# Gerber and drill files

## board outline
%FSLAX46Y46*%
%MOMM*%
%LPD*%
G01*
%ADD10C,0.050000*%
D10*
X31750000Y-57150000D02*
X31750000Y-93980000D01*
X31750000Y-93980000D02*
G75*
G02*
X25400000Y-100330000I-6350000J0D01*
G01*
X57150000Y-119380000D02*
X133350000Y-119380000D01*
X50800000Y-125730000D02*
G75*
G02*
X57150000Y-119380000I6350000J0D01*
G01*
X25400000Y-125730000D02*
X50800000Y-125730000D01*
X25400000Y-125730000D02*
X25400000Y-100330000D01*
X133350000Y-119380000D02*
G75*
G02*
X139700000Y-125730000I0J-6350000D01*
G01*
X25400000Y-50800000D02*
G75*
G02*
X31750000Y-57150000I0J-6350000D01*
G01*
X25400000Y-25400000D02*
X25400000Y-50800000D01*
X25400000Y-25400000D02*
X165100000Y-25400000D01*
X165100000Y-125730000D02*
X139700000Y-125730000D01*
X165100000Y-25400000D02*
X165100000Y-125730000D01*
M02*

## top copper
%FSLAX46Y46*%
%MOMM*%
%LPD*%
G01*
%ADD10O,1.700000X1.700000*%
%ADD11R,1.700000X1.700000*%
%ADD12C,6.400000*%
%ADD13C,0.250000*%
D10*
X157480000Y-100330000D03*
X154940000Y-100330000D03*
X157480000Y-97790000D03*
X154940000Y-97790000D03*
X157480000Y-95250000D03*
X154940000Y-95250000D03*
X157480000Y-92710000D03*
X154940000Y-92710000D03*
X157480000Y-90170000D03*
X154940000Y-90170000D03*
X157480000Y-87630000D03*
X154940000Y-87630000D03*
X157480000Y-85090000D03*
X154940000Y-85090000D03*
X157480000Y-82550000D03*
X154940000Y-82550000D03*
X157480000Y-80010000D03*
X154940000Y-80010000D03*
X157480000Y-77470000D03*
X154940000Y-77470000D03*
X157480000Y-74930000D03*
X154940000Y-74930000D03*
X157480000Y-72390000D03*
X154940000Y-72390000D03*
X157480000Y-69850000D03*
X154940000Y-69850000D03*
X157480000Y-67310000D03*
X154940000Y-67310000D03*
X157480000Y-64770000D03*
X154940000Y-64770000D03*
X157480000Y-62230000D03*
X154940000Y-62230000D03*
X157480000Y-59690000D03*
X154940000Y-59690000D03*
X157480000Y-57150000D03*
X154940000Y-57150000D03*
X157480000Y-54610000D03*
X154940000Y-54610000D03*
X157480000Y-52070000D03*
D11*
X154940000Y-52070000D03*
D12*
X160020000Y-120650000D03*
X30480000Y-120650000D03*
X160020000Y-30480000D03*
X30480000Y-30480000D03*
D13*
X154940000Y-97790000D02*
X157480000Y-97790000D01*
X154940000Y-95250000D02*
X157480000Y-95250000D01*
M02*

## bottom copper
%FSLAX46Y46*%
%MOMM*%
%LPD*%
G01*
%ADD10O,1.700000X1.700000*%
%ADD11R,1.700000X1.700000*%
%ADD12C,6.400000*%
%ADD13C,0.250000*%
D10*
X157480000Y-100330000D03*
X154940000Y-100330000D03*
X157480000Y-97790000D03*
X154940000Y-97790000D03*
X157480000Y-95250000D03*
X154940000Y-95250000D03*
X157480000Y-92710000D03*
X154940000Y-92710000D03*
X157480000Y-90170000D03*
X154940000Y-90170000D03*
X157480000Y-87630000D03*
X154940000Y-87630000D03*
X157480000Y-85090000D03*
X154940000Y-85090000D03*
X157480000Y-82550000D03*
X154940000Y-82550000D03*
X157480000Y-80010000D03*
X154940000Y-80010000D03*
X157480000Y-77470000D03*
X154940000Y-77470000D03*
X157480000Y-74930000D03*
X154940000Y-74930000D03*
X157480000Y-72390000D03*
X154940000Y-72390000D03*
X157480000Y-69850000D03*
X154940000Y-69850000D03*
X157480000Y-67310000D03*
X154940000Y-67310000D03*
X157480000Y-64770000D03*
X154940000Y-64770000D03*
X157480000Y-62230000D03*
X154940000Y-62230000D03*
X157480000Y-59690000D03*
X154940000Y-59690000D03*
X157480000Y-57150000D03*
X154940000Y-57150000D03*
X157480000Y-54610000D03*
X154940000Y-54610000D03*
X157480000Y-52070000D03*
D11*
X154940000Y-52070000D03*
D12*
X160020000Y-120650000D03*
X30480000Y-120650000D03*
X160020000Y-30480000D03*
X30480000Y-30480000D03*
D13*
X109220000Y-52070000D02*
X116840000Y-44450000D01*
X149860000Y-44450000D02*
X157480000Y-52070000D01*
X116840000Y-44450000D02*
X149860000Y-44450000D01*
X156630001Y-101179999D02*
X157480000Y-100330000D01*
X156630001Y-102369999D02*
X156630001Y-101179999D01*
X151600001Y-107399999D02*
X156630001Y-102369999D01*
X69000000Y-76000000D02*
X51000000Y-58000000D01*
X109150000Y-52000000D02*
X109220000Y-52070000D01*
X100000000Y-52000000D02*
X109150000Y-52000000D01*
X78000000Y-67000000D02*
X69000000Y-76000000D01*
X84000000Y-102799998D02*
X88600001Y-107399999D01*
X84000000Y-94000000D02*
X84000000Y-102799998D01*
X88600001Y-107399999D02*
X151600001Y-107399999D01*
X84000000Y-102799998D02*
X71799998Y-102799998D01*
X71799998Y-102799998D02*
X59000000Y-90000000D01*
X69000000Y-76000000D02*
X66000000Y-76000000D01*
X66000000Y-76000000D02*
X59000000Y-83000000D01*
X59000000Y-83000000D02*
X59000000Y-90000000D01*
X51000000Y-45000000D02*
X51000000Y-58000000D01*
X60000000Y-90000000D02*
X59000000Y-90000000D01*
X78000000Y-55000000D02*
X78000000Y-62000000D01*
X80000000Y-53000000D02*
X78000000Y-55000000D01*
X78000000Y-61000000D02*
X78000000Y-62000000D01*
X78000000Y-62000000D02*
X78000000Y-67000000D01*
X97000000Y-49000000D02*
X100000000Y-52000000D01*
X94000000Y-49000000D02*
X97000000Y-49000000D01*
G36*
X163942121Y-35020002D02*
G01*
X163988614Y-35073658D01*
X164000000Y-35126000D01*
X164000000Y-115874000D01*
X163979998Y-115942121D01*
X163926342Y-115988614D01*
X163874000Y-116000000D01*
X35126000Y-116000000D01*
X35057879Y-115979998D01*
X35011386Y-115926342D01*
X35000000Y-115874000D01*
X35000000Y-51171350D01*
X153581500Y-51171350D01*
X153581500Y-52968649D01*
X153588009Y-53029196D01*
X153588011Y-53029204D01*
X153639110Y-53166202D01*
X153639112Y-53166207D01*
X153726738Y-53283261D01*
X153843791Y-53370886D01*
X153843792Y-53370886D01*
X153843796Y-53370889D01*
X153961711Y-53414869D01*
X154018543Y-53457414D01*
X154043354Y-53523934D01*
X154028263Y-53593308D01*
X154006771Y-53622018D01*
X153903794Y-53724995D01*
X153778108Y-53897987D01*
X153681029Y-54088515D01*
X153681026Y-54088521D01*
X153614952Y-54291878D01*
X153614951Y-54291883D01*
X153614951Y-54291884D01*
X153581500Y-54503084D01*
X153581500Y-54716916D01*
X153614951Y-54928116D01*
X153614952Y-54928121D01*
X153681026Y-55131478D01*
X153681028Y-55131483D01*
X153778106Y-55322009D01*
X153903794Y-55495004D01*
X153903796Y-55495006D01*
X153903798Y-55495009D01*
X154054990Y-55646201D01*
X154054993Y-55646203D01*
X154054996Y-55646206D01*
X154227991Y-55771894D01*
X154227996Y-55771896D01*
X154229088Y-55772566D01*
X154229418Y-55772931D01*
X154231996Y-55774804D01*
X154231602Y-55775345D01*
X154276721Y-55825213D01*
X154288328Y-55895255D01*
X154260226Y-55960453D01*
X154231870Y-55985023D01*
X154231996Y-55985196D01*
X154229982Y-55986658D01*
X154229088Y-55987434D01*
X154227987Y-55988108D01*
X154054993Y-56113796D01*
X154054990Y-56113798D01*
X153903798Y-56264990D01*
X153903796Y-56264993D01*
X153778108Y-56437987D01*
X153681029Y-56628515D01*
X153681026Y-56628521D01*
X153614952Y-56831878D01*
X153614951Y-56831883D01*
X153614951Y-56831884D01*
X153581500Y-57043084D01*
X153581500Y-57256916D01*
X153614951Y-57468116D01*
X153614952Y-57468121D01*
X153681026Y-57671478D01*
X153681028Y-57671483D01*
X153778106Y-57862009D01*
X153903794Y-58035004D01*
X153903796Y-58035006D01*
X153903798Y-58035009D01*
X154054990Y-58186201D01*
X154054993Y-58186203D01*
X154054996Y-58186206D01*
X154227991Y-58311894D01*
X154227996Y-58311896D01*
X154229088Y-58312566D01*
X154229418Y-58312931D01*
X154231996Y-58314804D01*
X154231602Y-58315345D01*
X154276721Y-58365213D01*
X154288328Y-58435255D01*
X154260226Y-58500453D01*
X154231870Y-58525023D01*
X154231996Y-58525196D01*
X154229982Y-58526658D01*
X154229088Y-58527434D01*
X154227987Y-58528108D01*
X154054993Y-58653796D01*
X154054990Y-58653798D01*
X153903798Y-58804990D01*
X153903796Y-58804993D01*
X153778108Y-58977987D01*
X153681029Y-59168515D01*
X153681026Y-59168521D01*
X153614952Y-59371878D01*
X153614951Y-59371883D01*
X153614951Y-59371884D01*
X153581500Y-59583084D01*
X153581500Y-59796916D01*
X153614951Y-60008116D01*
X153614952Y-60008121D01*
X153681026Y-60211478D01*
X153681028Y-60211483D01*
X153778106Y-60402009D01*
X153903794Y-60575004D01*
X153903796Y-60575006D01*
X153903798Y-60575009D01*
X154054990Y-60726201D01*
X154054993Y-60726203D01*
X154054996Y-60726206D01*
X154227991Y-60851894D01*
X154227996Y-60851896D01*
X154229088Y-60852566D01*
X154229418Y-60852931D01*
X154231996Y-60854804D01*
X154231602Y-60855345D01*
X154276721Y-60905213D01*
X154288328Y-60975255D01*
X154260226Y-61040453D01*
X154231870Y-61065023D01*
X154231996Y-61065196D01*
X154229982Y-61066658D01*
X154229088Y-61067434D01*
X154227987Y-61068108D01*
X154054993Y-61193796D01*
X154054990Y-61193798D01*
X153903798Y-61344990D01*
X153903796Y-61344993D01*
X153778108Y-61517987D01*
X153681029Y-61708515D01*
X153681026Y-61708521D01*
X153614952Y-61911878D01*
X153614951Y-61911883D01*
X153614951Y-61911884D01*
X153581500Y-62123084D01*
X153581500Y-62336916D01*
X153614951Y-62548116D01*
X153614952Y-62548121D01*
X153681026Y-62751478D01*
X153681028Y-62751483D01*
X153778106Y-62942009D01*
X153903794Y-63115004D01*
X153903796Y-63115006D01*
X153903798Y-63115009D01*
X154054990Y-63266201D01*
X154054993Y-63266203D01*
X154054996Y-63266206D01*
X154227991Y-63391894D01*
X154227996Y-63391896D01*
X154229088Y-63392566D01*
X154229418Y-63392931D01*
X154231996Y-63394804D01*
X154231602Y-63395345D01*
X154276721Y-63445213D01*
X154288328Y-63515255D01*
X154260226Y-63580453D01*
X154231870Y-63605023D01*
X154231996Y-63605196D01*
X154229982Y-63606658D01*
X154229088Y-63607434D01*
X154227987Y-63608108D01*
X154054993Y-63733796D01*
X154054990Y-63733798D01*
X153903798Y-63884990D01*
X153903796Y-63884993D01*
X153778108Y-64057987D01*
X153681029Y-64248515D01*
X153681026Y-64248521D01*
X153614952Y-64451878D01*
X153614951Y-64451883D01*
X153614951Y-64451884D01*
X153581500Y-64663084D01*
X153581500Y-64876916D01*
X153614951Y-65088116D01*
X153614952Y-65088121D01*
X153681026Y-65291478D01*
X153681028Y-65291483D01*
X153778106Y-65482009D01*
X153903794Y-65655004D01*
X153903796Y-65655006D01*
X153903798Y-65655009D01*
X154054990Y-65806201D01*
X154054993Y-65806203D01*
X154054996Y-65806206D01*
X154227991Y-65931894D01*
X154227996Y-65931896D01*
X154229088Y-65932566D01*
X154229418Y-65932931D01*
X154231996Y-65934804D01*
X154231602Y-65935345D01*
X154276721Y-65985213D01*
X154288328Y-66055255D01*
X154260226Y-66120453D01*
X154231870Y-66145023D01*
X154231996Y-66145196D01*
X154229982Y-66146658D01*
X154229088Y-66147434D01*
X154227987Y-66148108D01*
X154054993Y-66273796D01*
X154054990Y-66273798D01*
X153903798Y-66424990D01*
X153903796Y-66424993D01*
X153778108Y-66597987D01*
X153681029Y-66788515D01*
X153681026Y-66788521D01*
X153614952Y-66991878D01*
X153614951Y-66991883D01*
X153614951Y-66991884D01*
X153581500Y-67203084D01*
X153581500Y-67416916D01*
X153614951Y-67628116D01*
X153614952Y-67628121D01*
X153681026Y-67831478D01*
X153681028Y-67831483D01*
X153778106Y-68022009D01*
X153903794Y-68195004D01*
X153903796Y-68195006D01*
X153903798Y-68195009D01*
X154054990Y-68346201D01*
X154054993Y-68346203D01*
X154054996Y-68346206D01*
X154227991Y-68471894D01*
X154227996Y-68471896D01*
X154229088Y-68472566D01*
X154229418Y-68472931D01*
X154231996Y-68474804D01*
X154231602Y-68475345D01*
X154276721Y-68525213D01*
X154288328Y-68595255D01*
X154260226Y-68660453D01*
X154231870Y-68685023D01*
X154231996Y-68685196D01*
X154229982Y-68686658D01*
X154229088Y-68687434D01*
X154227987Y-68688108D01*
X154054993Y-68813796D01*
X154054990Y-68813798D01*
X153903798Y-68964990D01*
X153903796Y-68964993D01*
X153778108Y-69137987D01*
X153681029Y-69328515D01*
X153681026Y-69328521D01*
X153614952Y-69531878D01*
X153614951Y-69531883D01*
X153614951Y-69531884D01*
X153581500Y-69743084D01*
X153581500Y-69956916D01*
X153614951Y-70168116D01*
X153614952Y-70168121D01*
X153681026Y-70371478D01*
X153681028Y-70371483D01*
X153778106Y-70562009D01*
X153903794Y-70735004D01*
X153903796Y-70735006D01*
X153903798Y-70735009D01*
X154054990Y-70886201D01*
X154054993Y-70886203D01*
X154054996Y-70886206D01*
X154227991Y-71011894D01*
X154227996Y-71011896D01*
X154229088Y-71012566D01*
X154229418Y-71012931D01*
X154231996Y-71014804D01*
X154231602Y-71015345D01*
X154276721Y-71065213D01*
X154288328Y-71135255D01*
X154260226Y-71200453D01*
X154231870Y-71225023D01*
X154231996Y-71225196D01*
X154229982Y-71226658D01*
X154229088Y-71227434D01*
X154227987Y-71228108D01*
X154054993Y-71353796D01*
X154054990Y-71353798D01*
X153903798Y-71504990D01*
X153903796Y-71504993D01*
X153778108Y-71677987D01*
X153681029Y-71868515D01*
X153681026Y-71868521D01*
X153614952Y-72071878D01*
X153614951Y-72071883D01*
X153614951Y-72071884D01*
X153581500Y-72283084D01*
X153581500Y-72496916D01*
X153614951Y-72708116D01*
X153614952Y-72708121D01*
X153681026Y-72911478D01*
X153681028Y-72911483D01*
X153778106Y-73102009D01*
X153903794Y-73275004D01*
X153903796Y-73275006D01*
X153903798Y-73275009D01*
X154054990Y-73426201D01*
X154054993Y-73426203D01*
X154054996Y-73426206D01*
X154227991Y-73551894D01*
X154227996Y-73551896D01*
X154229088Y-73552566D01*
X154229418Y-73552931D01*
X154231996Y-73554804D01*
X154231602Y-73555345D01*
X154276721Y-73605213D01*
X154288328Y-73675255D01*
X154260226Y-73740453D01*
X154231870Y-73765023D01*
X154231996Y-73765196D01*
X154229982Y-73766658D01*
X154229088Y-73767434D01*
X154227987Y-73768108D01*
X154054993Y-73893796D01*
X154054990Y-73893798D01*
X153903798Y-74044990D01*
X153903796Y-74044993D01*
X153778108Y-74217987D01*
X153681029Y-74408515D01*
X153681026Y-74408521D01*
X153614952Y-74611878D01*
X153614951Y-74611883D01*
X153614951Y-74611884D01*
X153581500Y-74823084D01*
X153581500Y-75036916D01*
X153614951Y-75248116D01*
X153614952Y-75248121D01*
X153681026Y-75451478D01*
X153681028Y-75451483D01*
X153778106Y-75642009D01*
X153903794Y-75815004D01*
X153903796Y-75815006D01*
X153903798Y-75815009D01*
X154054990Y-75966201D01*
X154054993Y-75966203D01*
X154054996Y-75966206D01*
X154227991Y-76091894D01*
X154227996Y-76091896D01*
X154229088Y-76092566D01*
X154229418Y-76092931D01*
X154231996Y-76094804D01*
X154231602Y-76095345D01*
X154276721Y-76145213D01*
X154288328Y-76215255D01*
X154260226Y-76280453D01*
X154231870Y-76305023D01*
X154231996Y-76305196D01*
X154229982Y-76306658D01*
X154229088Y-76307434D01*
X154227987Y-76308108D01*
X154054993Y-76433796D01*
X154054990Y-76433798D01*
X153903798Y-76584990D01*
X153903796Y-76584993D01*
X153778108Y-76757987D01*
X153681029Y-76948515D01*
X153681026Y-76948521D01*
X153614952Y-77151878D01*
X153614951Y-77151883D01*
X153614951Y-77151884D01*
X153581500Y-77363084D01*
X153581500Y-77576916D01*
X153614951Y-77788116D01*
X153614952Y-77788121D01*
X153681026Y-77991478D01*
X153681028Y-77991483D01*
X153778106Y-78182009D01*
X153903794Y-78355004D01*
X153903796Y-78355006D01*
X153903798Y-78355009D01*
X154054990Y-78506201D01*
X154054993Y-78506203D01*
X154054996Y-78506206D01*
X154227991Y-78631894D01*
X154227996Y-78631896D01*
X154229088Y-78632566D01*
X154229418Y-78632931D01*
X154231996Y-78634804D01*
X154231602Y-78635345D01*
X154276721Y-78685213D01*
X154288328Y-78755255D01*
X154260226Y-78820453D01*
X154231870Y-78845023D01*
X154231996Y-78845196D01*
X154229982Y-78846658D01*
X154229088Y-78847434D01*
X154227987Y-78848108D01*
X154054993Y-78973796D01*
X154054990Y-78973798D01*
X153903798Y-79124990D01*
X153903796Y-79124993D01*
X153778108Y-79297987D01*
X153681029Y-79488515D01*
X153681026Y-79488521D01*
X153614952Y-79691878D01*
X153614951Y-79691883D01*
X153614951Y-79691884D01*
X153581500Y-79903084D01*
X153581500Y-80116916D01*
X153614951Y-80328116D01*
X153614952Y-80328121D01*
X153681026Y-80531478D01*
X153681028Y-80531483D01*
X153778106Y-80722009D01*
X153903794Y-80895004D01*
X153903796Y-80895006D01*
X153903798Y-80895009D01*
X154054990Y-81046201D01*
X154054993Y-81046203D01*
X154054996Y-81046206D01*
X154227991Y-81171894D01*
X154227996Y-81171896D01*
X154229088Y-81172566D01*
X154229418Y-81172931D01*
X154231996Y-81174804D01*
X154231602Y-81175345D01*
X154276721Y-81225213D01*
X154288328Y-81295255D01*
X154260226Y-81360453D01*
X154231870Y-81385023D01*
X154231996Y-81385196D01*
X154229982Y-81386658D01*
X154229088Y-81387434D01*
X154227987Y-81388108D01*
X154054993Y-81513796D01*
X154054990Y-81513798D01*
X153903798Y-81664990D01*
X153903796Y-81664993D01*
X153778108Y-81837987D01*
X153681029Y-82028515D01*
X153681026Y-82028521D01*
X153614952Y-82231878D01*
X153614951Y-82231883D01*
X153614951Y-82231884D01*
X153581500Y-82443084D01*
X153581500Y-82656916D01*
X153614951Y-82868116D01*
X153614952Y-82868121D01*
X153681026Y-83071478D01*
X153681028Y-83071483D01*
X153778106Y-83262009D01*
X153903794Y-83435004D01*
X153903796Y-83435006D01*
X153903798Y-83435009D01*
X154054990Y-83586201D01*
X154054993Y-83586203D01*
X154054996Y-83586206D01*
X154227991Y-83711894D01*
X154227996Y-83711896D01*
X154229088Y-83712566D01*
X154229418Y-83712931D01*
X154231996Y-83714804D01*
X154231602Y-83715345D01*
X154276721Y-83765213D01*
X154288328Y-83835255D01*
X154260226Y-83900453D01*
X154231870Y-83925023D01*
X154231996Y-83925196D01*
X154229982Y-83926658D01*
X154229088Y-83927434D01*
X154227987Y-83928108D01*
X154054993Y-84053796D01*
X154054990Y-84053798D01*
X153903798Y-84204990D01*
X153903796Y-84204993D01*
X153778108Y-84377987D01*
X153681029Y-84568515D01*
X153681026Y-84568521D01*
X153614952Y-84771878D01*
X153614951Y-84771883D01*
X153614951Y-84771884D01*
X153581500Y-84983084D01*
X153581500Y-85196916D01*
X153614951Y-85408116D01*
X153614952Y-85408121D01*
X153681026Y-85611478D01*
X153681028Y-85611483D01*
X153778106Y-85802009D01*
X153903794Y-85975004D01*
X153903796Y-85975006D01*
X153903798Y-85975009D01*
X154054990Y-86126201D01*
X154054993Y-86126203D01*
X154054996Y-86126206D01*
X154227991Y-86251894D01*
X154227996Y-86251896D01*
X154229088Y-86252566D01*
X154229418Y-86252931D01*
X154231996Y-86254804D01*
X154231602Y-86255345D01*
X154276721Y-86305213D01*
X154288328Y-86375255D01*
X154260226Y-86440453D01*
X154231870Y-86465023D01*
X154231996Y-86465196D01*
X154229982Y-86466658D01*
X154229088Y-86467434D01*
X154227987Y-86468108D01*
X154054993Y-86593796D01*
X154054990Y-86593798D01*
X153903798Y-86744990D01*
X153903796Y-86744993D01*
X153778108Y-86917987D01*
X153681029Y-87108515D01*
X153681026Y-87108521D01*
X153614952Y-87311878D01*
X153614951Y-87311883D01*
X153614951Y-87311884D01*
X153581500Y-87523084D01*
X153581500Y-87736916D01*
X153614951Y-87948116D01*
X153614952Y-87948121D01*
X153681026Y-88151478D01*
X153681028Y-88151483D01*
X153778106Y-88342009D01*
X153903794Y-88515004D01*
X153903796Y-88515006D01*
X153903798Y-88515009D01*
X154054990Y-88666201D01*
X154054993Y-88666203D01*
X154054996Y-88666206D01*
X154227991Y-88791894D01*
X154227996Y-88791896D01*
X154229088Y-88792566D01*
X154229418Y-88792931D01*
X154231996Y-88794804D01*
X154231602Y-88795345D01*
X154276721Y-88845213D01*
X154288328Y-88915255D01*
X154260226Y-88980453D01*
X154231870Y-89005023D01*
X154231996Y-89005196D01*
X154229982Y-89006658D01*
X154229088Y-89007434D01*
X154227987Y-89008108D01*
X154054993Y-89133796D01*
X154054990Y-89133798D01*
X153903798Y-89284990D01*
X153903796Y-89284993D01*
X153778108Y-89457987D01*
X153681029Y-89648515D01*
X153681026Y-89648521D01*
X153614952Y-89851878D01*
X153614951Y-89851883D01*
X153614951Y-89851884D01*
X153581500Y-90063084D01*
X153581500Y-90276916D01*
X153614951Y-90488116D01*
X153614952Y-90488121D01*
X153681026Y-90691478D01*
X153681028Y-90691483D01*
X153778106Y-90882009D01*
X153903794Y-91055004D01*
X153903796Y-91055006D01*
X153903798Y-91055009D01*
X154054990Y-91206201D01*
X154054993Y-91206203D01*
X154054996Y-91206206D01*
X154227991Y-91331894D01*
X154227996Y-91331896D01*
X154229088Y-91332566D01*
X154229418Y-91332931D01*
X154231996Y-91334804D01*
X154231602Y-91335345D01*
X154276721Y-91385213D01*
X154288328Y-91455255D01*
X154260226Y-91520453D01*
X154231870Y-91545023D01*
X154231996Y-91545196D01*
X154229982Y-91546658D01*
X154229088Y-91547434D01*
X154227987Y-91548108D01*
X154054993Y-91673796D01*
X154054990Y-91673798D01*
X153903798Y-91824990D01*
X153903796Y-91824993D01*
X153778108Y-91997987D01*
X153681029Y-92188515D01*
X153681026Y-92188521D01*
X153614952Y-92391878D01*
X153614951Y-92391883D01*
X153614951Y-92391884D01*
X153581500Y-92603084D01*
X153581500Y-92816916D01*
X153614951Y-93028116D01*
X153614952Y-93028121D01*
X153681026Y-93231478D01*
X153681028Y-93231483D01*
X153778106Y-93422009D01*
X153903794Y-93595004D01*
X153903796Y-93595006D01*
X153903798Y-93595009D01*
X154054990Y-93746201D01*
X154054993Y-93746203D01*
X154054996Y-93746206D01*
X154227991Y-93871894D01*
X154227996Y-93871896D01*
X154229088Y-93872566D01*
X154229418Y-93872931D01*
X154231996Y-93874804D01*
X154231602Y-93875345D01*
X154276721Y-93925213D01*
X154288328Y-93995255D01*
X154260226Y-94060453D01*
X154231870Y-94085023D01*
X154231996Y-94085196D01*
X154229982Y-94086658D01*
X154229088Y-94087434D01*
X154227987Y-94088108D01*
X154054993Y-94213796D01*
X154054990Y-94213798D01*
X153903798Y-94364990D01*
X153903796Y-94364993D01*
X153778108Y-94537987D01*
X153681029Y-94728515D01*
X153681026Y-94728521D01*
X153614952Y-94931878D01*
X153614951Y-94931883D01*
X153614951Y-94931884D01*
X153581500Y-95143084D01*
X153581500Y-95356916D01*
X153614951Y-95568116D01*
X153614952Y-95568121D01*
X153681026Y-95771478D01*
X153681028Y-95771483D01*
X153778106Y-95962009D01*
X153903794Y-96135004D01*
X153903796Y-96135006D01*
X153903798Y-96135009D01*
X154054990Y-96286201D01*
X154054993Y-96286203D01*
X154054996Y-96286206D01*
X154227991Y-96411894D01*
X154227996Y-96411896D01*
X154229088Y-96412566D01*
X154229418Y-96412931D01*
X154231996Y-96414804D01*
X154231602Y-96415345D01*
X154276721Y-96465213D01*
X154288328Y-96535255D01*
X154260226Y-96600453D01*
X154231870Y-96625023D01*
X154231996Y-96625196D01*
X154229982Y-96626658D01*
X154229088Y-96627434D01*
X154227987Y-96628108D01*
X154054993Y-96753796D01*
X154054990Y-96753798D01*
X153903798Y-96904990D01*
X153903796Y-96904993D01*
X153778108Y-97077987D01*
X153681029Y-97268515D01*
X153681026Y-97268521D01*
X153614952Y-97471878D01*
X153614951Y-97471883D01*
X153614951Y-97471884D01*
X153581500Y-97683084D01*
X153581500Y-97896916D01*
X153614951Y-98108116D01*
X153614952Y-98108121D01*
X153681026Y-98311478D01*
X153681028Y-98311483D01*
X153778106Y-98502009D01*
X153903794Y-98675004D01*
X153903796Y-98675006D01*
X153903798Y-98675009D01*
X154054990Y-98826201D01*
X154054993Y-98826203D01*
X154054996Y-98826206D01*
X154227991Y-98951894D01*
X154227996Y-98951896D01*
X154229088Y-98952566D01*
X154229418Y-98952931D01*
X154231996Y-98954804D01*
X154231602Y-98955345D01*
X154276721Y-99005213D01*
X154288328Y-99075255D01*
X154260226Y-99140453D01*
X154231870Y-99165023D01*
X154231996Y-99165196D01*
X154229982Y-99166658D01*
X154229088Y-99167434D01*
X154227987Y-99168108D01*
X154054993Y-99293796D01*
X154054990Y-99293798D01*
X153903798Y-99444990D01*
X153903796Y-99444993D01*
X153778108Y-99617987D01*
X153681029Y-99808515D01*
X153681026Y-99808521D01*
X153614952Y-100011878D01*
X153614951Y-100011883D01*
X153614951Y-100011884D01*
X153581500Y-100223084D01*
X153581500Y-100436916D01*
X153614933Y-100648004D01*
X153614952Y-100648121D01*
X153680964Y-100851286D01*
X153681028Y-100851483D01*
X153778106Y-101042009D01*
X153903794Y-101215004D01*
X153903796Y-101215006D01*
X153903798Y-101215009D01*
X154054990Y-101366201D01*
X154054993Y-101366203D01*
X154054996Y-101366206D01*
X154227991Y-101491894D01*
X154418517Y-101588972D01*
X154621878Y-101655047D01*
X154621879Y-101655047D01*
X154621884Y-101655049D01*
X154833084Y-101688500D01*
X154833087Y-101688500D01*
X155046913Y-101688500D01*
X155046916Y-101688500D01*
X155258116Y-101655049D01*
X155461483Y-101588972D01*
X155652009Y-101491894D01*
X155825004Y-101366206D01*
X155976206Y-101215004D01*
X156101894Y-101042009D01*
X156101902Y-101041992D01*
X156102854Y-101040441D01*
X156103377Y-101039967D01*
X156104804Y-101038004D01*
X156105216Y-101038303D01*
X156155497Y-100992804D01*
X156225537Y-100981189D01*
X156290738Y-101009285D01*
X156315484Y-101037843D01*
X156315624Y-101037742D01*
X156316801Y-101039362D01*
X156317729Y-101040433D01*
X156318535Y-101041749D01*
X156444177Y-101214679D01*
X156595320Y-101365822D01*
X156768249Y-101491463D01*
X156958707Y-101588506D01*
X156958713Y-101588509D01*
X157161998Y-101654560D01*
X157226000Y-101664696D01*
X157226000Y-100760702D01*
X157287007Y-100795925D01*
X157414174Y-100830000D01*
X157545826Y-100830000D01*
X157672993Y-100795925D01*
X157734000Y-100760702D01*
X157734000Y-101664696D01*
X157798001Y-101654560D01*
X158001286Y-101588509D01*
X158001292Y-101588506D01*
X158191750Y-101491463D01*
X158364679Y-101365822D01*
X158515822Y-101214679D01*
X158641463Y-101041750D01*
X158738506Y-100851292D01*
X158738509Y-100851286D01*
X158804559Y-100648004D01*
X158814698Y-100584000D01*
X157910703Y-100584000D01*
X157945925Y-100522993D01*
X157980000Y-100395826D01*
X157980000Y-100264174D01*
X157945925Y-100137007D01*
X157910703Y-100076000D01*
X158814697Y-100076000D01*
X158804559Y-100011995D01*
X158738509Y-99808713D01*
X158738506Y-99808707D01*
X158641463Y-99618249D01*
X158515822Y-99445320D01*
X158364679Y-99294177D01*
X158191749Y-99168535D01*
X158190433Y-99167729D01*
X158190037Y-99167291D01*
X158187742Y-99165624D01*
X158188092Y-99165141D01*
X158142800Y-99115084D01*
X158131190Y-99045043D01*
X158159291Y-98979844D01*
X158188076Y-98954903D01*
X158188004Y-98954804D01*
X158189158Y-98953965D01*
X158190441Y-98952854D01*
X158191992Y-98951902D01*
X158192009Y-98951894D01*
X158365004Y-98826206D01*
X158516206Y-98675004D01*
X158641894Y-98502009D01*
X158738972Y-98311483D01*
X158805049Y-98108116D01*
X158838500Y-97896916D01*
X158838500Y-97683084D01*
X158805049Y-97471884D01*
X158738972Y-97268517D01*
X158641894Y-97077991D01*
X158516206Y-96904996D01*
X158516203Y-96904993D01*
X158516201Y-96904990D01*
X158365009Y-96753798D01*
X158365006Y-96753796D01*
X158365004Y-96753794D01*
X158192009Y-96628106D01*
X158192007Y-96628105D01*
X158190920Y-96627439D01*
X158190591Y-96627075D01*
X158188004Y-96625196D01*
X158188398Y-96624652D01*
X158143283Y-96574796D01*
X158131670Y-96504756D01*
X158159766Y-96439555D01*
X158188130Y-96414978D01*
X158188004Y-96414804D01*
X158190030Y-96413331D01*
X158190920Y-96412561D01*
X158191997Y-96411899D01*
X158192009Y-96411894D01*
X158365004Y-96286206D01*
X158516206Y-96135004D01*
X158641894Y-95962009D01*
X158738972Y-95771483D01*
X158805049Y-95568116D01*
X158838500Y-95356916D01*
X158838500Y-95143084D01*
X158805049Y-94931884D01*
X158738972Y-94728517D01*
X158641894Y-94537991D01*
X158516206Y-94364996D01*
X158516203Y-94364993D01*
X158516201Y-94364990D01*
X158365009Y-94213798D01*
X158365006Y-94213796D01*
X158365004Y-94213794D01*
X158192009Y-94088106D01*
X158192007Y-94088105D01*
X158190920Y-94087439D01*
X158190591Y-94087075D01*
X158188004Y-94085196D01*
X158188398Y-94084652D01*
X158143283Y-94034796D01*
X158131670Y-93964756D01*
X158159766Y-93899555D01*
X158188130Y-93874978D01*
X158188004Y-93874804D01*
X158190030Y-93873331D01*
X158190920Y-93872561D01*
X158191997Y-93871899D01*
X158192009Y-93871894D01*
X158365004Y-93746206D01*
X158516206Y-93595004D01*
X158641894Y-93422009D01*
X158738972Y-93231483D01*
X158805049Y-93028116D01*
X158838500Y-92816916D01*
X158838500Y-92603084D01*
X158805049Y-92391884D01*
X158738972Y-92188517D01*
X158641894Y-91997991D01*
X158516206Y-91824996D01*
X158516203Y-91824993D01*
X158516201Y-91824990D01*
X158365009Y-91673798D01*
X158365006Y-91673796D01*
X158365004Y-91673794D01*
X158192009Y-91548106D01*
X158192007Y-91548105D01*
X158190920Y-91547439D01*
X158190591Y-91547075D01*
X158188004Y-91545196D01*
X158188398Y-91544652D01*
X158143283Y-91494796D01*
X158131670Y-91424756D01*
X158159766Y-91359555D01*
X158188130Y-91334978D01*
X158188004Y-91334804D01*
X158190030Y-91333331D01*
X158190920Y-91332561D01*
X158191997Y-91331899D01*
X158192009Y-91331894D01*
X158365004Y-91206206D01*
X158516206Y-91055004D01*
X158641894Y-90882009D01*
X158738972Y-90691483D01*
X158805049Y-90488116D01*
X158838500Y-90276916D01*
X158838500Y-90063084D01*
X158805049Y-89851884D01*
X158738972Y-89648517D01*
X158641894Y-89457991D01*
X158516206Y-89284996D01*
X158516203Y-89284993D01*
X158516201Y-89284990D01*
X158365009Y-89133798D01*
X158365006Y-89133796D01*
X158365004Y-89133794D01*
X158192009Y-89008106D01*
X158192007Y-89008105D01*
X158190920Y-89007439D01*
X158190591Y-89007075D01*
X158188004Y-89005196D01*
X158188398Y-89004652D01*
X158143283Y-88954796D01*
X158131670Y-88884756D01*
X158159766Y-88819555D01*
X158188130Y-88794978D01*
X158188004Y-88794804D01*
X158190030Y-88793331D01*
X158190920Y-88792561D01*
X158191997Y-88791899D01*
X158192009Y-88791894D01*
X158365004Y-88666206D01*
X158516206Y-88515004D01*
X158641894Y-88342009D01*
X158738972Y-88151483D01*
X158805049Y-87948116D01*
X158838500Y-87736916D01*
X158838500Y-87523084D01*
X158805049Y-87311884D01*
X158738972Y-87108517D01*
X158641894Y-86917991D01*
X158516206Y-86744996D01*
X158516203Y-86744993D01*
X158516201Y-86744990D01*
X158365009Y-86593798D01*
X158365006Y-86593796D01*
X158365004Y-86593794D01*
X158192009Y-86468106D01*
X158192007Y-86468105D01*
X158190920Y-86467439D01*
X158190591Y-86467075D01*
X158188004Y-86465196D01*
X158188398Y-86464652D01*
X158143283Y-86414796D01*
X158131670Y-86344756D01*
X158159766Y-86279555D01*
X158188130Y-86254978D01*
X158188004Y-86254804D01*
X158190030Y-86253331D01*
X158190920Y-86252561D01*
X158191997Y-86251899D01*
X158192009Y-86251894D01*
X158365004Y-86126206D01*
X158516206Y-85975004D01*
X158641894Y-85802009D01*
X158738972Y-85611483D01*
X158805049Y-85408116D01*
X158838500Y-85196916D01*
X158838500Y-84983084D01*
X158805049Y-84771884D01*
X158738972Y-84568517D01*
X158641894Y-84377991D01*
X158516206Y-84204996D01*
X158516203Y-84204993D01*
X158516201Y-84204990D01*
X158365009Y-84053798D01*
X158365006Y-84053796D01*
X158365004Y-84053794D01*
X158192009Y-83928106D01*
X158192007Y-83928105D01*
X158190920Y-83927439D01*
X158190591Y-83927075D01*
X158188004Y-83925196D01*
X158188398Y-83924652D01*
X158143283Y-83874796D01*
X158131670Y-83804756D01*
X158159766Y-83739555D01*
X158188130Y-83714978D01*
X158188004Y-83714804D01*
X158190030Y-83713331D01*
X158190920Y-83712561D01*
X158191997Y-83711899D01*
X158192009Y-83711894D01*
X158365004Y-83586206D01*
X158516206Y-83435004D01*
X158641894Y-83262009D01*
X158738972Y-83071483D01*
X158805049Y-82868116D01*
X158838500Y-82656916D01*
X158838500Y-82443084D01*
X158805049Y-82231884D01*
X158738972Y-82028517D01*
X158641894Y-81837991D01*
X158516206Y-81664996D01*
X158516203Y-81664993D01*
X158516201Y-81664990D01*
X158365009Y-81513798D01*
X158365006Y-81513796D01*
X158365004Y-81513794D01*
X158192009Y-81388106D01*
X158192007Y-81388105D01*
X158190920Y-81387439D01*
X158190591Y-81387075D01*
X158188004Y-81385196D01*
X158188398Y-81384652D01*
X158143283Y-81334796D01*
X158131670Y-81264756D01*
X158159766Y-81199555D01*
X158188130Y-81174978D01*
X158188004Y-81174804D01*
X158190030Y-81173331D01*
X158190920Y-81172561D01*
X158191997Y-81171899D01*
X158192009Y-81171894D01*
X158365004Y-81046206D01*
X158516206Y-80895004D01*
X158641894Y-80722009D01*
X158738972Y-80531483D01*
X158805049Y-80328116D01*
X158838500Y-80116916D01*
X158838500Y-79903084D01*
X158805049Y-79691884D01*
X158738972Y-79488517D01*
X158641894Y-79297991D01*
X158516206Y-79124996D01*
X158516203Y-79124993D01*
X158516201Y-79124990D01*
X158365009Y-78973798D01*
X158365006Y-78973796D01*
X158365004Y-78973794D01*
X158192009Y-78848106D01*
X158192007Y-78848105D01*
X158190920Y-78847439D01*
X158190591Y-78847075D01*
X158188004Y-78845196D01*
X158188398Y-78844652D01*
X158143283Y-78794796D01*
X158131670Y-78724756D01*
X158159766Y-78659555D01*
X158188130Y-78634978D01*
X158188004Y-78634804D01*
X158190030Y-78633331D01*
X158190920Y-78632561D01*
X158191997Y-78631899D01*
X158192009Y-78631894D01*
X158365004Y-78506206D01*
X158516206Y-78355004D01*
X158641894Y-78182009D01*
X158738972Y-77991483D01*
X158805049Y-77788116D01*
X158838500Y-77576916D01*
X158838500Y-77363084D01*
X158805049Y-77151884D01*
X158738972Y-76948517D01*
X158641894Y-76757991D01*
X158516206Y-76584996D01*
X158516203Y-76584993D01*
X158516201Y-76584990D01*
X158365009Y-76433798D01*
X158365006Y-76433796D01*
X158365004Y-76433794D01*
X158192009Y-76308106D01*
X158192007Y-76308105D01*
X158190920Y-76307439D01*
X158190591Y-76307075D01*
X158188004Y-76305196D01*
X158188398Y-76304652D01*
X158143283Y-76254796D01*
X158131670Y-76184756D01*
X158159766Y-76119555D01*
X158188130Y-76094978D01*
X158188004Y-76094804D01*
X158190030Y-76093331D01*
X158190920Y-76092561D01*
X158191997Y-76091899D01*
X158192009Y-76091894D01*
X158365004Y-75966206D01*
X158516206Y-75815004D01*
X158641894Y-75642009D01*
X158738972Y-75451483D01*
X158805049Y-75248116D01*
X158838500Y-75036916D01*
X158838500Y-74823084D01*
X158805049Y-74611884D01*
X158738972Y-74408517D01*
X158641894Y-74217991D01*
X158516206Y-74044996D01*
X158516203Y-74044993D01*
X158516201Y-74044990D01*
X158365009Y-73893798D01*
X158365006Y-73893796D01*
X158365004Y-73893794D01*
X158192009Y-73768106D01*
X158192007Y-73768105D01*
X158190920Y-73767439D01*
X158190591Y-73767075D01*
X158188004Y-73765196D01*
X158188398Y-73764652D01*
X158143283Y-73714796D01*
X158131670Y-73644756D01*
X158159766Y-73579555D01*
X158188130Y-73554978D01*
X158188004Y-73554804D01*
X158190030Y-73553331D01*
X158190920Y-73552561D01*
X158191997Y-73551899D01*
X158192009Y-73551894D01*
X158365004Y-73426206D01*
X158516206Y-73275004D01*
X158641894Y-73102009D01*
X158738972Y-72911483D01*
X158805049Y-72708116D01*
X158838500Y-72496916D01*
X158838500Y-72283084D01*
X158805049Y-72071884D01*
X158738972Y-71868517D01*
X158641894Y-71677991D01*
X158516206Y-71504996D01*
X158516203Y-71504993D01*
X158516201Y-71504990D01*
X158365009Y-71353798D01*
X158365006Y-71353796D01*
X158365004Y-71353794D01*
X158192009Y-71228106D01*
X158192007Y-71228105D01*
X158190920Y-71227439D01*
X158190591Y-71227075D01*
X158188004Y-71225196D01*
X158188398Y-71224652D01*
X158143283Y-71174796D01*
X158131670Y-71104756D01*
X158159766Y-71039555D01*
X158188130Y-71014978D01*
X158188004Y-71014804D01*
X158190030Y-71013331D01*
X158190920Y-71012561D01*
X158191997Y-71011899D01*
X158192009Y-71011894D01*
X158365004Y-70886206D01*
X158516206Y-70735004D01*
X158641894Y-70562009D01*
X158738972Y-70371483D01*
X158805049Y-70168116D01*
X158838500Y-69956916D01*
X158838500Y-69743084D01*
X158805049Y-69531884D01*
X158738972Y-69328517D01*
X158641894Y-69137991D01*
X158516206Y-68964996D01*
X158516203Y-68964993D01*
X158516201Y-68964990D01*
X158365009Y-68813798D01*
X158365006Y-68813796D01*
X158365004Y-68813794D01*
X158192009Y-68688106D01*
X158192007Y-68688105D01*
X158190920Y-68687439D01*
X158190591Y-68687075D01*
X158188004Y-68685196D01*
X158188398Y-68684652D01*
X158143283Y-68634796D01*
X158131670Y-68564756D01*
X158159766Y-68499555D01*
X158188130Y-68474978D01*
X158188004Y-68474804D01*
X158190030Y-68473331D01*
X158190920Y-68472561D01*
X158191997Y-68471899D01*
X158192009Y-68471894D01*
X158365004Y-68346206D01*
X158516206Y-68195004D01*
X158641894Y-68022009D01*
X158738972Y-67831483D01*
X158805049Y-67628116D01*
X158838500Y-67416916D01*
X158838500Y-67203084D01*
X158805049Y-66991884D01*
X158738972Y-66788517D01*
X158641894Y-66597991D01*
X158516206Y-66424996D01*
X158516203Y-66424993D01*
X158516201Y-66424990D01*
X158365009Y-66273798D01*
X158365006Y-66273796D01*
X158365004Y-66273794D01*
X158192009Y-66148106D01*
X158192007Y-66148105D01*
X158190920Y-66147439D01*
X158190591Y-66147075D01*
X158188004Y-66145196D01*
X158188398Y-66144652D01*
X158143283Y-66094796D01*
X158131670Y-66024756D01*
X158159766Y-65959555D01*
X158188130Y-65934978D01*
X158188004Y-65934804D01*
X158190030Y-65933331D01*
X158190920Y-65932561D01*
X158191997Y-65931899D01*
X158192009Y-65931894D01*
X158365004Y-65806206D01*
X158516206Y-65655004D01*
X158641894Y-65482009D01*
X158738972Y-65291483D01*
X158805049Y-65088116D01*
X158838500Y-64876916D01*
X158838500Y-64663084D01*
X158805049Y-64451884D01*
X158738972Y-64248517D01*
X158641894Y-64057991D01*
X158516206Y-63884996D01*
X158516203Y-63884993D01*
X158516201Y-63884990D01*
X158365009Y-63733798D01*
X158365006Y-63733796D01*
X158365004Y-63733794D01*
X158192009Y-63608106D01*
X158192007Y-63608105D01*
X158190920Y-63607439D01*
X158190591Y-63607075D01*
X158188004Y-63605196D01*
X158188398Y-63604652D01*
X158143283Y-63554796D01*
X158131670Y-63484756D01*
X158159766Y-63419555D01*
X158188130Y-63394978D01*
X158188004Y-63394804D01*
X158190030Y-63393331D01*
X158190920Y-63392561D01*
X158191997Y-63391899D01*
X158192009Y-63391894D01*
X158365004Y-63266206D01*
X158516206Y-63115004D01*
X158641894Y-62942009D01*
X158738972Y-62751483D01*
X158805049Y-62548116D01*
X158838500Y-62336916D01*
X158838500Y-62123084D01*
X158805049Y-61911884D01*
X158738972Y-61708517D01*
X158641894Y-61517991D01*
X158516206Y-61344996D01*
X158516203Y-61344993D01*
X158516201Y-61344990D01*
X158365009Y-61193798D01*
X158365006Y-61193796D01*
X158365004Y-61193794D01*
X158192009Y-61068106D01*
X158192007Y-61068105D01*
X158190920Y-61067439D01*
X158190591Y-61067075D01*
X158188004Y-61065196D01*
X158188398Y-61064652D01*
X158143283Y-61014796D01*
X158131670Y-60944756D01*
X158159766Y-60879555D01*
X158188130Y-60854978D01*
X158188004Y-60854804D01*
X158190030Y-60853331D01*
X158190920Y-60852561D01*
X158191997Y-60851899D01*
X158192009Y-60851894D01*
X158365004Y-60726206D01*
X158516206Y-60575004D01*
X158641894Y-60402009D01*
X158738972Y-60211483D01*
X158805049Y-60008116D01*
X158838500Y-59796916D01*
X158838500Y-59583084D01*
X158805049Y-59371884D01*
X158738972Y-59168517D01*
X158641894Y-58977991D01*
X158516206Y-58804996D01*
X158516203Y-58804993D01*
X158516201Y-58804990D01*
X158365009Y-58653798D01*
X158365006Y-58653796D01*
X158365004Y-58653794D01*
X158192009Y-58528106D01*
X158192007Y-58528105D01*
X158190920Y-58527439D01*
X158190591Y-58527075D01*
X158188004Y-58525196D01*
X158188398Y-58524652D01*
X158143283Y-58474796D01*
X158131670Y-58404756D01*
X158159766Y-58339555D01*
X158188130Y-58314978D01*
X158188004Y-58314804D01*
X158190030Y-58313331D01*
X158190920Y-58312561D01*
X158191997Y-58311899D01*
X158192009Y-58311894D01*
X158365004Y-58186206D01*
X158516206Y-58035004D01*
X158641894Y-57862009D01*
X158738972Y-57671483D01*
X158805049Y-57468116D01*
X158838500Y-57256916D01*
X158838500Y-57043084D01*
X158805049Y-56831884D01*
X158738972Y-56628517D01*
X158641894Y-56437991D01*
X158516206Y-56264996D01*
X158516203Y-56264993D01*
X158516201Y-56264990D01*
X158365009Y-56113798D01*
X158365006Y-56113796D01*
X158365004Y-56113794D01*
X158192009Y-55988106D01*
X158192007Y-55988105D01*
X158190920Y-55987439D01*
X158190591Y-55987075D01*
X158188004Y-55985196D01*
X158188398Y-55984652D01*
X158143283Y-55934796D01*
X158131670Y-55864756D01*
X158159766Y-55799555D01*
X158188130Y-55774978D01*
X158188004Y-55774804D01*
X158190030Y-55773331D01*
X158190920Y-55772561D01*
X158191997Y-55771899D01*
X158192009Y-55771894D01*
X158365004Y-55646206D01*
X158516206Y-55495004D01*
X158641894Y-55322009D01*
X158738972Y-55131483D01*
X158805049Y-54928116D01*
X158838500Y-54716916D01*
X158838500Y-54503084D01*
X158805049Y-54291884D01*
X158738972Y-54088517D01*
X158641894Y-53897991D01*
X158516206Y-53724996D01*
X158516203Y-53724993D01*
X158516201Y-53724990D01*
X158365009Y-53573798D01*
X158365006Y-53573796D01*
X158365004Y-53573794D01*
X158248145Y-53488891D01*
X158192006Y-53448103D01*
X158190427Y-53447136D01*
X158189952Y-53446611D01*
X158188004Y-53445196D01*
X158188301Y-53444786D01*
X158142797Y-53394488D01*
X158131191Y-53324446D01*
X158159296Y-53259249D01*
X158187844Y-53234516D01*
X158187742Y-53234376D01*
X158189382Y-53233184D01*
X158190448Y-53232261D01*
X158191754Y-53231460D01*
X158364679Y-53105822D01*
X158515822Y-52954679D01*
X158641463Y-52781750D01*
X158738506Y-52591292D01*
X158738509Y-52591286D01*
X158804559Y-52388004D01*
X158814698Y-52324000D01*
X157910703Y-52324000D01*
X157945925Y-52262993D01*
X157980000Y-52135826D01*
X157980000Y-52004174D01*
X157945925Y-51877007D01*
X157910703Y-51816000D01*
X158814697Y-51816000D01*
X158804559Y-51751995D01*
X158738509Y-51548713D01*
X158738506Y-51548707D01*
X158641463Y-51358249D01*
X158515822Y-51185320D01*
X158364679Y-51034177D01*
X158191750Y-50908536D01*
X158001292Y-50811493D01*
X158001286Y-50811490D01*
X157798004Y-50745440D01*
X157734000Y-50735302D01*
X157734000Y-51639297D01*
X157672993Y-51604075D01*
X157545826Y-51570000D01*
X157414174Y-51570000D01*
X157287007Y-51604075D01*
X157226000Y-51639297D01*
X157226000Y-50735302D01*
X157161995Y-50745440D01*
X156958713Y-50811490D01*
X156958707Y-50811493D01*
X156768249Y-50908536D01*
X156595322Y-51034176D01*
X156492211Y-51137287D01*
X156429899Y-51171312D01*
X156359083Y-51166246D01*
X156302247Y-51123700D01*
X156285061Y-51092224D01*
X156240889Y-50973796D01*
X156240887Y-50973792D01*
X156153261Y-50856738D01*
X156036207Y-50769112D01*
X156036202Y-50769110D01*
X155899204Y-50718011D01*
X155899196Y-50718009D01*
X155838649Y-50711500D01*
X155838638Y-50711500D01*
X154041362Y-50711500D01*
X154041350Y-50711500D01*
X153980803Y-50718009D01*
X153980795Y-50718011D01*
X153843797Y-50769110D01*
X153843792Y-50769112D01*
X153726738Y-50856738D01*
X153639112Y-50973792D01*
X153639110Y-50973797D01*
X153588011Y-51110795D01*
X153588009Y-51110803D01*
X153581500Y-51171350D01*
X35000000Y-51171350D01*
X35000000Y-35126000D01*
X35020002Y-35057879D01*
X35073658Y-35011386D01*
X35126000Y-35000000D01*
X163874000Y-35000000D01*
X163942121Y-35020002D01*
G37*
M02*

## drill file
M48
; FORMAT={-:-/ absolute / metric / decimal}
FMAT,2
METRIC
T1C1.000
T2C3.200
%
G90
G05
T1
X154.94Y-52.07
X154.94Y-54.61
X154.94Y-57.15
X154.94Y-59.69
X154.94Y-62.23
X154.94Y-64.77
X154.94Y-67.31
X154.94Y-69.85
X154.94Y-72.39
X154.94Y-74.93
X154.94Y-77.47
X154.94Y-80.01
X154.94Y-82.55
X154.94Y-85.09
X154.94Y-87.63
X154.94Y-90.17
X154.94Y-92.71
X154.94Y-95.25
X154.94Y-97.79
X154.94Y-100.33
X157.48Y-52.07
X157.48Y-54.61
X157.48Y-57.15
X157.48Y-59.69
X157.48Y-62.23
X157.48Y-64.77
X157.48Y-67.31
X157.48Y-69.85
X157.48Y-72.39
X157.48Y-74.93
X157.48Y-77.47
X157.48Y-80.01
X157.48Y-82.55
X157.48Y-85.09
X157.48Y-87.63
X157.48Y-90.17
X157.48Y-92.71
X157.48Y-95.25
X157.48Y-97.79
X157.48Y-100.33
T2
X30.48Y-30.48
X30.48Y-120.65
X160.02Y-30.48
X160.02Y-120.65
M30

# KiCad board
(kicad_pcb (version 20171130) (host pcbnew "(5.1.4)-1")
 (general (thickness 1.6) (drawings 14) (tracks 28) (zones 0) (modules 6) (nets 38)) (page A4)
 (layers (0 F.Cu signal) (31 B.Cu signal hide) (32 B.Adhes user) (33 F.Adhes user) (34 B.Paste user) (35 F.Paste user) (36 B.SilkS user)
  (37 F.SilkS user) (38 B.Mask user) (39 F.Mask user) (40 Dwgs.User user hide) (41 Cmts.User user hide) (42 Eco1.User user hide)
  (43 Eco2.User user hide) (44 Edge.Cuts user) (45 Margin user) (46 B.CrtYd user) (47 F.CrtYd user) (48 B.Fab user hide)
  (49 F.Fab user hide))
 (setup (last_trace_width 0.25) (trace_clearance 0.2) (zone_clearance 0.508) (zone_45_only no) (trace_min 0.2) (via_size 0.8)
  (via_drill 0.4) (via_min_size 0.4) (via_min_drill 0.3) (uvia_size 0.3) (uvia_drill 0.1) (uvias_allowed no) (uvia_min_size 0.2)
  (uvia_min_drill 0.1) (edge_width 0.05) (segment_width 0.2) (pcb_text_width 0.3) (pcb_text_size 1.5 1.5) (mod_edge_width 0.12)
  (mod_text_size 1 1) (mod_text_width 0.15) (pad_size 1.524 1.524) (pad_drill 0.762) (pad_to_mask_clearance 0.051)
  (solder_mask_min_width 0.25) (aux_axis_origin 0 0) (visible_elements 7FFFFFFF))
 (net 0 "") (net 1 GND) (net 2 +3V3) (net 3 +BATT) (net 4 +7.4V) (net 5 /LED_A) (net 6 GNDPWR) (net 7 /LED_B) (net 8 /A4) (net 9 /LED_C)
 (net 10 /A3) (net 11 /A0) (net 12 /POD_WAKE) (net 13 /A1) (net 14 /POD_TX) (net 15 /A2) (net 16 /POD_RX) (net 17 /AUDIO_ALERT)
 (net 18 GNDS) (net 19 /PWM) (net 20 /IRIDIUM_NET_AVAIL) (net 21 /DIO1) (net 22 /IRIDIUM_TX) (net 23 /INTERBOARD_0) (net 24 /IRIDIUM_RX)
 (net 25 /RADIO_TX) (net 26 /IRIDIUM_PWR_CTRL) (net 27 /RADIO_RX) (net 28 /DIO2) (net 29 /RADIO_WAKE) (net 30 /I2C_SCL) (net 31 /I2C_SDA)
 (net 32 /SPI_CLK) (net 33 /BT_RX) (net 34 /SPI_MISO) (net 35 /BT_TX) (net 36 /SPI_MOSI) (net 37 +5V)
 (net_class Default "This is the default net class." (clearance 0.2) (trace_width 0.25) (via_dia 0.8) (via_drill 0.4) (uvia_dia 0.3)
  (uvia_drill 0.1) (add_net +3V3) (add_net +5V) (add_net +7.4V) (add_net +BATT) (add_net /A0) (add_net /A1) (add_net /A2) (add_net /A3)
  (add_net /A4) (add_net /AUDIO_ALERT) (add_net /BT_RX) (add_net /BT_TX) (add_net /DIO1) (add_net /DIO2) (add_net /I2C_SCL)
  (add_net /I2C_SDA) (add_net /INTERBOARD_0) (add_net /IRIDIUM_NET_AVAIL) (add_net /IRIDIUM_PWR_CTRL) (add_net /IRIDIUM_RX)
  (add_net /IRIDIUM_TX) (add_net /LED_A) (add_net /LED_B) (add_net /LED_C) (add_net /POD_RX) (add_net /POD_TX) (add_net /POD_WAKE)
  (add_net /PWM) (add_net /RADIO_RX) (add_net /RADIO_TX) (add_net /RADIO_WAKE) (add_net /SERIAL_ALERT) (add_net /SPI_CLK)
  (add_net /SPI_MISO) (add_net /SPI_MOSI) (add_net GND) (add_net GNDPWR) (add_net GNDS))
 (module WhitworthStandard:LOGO (layer F.Cu) (at 58 32)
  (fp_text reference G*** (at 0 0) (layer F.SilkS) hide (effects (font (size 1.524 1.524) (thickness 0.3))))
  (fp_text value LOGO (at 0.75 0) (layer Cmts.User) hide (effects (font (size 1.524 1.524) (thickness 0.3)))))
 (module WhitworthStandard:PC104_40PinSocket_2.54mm (layer F.Cu) (at 154.94 52.07)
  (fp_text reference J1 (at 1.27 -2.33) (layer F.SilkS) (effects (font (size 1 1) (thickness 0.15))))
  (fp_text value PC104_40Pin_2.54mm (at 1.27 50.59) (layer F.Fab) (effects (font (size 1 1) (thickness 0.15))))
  (pad 21 thru_hole oval (at 2.54 48.26) (size 1.7 1.7) (drill 1) (layers *.Cu *.Mask) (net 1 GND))
  (pad 20 thru_hole oval (at 0 48.26) (size 1.7 1.7) (drill 1) (layers *.Cu *.Mask) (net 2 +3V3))
  (pad 22 thru_hole oval (at 2.54 45.72) (size 1.7 1.7) (drill 1) (layers *.Cu *.Mask) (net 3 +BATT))
  (pad 19 thru_hole oval (at 0 45.72) (size 1.7 1.7) (drill 1) (layers *.Cu *.Mask) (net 3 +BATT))
  (pad 23 thru_hole oval (at 2.54 43.18) (size 1.7 1.7) (drill 1) (layers *.Cu *.Mask) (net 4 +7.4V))
  (pad 18 thru_hole oval (at 0 43.18) (size 1.7 1.7) (drill 1) (layers *.Cu *.Mask) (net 4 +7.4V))
  (pad 24 thru_hole oval (at 2.54 40.64) (size 1.7 1.7) (drill 1) (layers *.Cu *.Mask) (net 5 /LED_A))
  (pad 17 thru_hole oval (at 0 40.64) (size 1.7 1.7) (drill 1) (layers *.Cu *.Mask) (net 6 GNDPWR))
  (pad 25 thru_hole oval (at 2.54 38.1) (size 1.7 1.7) (drill 1) (layers *.Cu *.Mask) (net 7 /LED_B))
  (pad 16 thru_hole oval (at 0 38.1) (size 1.7 1.7) (drill 1) (layers *.Cu *.Mask) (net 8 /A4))
  (pad 26 thru_hole oval (at 2.54 35.56) (size 1.7 1.7) (drill 1) (layers *.Cu *.Mask) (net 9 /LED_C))
  (pad 15 thru_hole oval (at 0 35.56) (size 1.7 1.7) (drill 1) (layers *.Cu *.Mask) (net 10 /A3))
  (pad 27 thru_hole oval (at 2.54 33.02) (size 1.7 1.7) (drill 1) (layers *.Cu *.Mask) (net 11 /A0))
  (pad 14 thru_hole oval (at 0 33.02) (size 1.7 1.7) (drill 1) (layers *.Cu *.Mask) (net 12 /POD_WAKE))
  (pad 28 thru_hole oval (at 2.54 30.48) (size 1.7 1.7) (drill 1) (layers *.Cu *.Mask) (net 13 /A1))
  (pad 13 thru_hole oval (at 0 30.48) (size 1.7 1.7) (drill 1) (layers *.Cu *.Mask) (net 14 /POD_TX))
  (pad 29 thru_hole oval (at 2.54 27.94) (size 1.7 1.7) (drill 1) (layers *.Cu *.Mask) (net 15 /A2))
  (pad 12 thru_hole oval (at 0 27.94) (size 1.7 1.7) (drill 1) (layers *.Cu *.Mask) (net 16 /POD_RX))
  (pad 30 thru_hole oval (at 2.54 25.4) (size 1.7 1.7) (drill 1) (layers *.Cu *.Mask) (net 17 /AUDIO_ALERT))
  (pad 11 thru_hole oval (at 0 25.4) (size 1.7 1.7) (drill 1) (layers *.Cu *.Mask) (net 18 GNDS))
  (pad 31 thru_hole oval (at 2.54 22.86) (size 1.7 1.7) (drill 1) (layers *.Cu *.Mask) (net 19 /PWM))
  (pad 10 thru_hole oval (at 0 22.86) (size 1.7 1.7) (drill 1) (layers *.Cu *.Mask) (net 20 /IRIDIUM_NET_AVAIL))
  (pad 32 thru_hole oval (at 2.54 20.32) (size 1.7 1.7) (drill 1) (layers *.Cu *.Mask) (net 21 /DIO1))
  (pad 9 thru_hole oval (at 0 20.32) (size 1.7 1.7) (drill 1) (layers *.Cu *.Mask) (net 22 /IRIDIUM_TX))
  (pad 33 thru_hole oval (at 2.54 17.78) (size 1.7 1.7) (drill 1) (layers *.Cu *.Mask) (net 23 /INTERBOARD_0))
  (pad 8 thru_hole oval (at 0 17.78) (size 1.7 1.7) (drill 1) (layers *.Cu *.Mask) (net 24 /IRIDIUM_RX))
  (pad 34 thru_hole oval (at 2.54 15.24) (size 1.7 1.7) (drill 1) (layers *.Cu *.Mask) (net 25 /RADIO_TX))
  (pad 7 thru_hole oval (at 0 15.24) (size 1.7 1.7) (drill 1) (layers *.Cu *.Mask) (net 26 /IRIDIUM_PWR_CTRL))
  (pad 35 thru_hole oval (at 2.54 12.7) (size 1.7 1.7) (drill 1) (layers *.Cu *.Mask) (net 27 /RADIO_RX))
  (pad 6 thru_hole oval (at 0 12.7) (size 1.7 1.7) (drill 1) (layers *.Cu *.Mask) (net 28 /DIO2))
  (pad 36 thru_hole oval (at 2.54 10.16) (size 1.7 1.7) (drill 1) (layers *.Cu *.Mask) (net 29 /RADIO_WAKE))
  (pad 5 thru_hole oval (at 0 10.16) (size 1.7 1.7) (drill 1) (layers *.Cu *.Mask) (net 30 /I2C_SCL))
  (pad 37 thru_hole oval (at 2.54 7.62) (size 1.7 1.7) (drill 1) (layers *.Cu *.Mask) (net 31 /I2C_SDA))
  (pad 4 thru_hole oval (at 0 7.62) (size 1.7 1.7) (drill 1) (layers *.Cu *.Mask) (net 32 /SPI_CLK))
  (pad 38 thru_hole oval (at 2.54 5.08) (size 1.7 1.7) (drill 1) (layers *.Cu *.Mask) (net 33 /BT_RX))
  (pad 3 thru_hole oval (at 0 5.08) (size 1.7 1.7) (drill 1) (layers *.Cu *.Mask) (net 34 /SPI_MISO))
  (pad 39 thru_hole oval (at 2.54 2.54) (size 1.7 1.7) (drill 1) (layers *.Cu *.Mask) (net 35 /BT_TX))
  (pad 2 thru_hole oval (at 0 2.54) (size 1.7 1.7) (drill 1) (layers *.Cu *.Mask) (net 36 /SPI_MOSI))
  (pad 40 thru_hole oval (at 2.54 0) (size 1.7 1.7) (drill 1) (layers *.Cu *.Mask) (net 1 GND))
  (pad 1 thru_hole rect (at 0 0) (size 1.7 1.7) (drill 1) (layers *.Cu *.Mask) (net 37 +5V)))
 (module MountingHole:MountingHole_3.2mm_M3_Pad (layer F.Cu) (at 160.02 120.65)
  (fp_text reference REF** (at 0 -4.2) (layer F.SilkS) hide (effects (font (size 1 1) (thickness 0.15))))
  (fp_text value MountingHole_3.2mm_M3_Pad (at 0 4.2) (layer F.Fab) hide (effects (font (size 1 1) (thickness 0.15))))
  (pad 1 thru_hole circle (at 0 0) (size 6.4 6.4) (drill 3.2) (layers *.Cu *.Mask)))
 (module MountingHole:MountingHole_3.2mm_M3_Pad (layer F.Cu) (at 30.48 120.65)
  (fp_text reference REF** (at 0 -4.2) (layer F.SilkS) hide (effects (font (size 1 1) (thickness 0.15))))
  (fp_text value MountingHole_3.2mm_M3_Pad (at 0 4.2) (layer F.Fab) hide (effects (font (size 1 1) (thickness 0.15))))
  (pad 1 thru_hole circle (at 0 0) (size 6.4 6.4) (drill 3.2) (layers *.Cu *.Mask)))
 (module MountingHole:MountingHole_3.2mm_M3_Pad (layer F.Cu) (at 160.02 30.48)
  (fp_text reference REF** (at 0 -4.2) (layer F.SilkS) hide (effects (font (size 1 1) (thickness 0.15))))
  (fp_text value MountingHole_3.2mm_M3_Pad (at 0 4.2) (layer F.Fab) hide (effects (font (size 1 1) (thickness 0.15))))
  (pad 1 thru_hole circle (at 0 0) (size 6.4 6.4) (drill 3.2) (layers *.Cu *.Mask)))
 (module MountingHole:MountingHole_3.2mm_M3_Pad (layer F.Cu) (at 30.48 30.48)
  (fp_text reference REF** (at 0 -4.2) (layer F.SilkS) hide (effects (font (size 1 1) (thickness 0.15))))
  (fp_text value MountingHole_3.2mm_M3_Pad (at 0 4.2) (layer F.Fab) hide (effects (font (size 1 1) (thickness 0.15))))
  (pad 1 thru_hole circle (at 0 0) (size 6.4 6.4) (drill 3.2) (layers *.Cu *.Mask)))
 (gr_line (start 31.75 57.15) (end 31.75 93.98) (layer Edge.Cuts) (width 0.05))
 (gr_arc (start 25.4 93.98) (end 25.4 100.33) (angle -90) (layer Edge.Cuts) (width 0.05))
 (gr_line (start 57.15 119.38) (end 133.35 119.38) (layer Edge.Cuts) (width 0.05))
 (gr_arc (start 57.15 125.73) (end 57.15 119.38) (angle -90) (layer Edge.Cuts) (width 0.05))
 (gr_line (start 25.4 125.73) (end 50.8 125.73) (layer Edge.Cuts) (width 0.05))
 (gr_line (start 25.4 125.73) (end 25.4 100.33) (layer Edge.Cuts) (width 0.05))
 (gr_arc (start 133.35 125.73) (end 139.7 125.73) (angle -90) (layer Edge.Cuts) (width 0.05))
 (gr_arc (start 25.4 57.15) (end 31.75 57.15) (angle -90) (layer Edge.Cuts) (width 0.05))
 (gr_line (start 25.4 25.4) (end 25.4 50.8) (layer Edge.Cuts) (width 0.05))
 (gr_line (start 25.4 25.4) (end 165.1 25.4) (layer Edge.Cuts) (width 0.05))
 (gr_line (start 165.1 125.73) (end 139.7 125.73) (layer Edge.Cuts) (width 0.05))
 (gr_line (start 165.1 25.4) (end 165.1 125.73) (layer Edge.Cuts) (width 0.05))
 (segment (start 109.22 52.07) (end 116.84 44.45) (width 0.25) (layer B.Cu) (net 1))
 (segment (start 149.86 44.45) (end 157.48 52.07) (width 0.25) (layer B.Cu) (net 1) (status 20))
 (segment (start 116.84 44.45) (end 149.86 44.45) (width 0.25) (layer B.Cu) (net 1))
 (segment (start 156.630001 101.179999) (end 157.48 100.33) (width 0.25) (layer B.Cu) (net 1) (status 20))
 (segment (start 156.630001 102.369999) (end 156.630001 101.179999) (width 0.25) (layer B.Cu) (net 1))
 (segment (start 151.600001 107.399999) (end 156.630001 102.369999) (width 0.25) (layer B.Cu) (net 1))
 (segment (start 69 76) (end 51 58) (width 0.25) (layer B.Cu) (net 1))
 (segment (start 109.15 52) (end 109.22 52.07) (width 0.25) (layer B.Cu) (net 1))
 (segment (start 100 52) (end 109.15 52) (width 0.25) (layer B.Cu) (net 1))
 (segment (start 78 67) (end 69 76) (width 0.25) (layer B.Cu) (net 1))
 (segment (start 84 102.799998) (end 88.600001 107.399999) (width 0.25) (layer B.Cu) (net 1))
 (segment (start 84 94) (end 84 102.799998) (width 0.25) (layer B.Cu) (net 1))
 (segment (start 88.600001 107.399999) (end 151.600001 107.399999) (width 0.25) (layer B.Cu) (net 1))
 (segment (start 84 102.799998) (end 71.799998 102.799998) (width 0.25) (layer B.Cu) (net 1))
 (segment (start 71.799998 102.799998) (end 59 90) (width 0.25) (layer B.Cu) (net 1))
 (segment (start 69 76) (end 66 76) (width 0.25) (layer B.Cu) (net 1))
 (segment (start 66 76) (end 59 83) (width 0.25) (layer B.Cu) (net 1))
 (segment (start 59 83) (end 59 90) (width 0.25) (layer B.Cu) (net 1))
 (segment (start 51 45) (end 51 58) (width 0.25) (layer B.Cu) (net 1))
 (segment (start 60 90) (end 59 90) (width 0.25) (layer B.Cu) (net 1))
 (segment (start 78 55) (end 78 62) (width 0.25) (layer B.Cu) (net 1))
 (segment (start 80 53) (end 78 55) (width 0.25) (layer B.Cu) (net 1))
 (segment (start 78 61) (end 78 62) (width 0.25) (layer B.Cu) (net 1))
 (segment (start 78 62) (end 78 67) (width 0.25) (layer B.Cu) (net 1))
 (segment (start 97 49) (end 100 52) (width 0.25) (layer B.Cu) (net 1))
 (segment (start 94 49) (end 97 49) (width 0.25) (layer B.Cu) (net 1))
 (segment (start 154.94 97.79) (end 157.48 97.79) (width 0.25) (layer F.Cu) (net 3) (status 30))
 (segment (start 154.94 95.25) (end 157.48 95.25) (width 0.25) (layer F.Cu) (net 4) (status 30))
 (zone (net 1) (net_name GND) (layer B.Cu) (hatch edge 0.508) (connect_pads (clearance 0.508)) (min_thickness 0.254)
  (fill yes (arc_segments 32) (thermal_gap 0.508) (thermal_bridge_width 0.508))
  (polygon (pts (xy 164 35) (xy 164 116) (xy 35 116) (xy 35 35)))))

